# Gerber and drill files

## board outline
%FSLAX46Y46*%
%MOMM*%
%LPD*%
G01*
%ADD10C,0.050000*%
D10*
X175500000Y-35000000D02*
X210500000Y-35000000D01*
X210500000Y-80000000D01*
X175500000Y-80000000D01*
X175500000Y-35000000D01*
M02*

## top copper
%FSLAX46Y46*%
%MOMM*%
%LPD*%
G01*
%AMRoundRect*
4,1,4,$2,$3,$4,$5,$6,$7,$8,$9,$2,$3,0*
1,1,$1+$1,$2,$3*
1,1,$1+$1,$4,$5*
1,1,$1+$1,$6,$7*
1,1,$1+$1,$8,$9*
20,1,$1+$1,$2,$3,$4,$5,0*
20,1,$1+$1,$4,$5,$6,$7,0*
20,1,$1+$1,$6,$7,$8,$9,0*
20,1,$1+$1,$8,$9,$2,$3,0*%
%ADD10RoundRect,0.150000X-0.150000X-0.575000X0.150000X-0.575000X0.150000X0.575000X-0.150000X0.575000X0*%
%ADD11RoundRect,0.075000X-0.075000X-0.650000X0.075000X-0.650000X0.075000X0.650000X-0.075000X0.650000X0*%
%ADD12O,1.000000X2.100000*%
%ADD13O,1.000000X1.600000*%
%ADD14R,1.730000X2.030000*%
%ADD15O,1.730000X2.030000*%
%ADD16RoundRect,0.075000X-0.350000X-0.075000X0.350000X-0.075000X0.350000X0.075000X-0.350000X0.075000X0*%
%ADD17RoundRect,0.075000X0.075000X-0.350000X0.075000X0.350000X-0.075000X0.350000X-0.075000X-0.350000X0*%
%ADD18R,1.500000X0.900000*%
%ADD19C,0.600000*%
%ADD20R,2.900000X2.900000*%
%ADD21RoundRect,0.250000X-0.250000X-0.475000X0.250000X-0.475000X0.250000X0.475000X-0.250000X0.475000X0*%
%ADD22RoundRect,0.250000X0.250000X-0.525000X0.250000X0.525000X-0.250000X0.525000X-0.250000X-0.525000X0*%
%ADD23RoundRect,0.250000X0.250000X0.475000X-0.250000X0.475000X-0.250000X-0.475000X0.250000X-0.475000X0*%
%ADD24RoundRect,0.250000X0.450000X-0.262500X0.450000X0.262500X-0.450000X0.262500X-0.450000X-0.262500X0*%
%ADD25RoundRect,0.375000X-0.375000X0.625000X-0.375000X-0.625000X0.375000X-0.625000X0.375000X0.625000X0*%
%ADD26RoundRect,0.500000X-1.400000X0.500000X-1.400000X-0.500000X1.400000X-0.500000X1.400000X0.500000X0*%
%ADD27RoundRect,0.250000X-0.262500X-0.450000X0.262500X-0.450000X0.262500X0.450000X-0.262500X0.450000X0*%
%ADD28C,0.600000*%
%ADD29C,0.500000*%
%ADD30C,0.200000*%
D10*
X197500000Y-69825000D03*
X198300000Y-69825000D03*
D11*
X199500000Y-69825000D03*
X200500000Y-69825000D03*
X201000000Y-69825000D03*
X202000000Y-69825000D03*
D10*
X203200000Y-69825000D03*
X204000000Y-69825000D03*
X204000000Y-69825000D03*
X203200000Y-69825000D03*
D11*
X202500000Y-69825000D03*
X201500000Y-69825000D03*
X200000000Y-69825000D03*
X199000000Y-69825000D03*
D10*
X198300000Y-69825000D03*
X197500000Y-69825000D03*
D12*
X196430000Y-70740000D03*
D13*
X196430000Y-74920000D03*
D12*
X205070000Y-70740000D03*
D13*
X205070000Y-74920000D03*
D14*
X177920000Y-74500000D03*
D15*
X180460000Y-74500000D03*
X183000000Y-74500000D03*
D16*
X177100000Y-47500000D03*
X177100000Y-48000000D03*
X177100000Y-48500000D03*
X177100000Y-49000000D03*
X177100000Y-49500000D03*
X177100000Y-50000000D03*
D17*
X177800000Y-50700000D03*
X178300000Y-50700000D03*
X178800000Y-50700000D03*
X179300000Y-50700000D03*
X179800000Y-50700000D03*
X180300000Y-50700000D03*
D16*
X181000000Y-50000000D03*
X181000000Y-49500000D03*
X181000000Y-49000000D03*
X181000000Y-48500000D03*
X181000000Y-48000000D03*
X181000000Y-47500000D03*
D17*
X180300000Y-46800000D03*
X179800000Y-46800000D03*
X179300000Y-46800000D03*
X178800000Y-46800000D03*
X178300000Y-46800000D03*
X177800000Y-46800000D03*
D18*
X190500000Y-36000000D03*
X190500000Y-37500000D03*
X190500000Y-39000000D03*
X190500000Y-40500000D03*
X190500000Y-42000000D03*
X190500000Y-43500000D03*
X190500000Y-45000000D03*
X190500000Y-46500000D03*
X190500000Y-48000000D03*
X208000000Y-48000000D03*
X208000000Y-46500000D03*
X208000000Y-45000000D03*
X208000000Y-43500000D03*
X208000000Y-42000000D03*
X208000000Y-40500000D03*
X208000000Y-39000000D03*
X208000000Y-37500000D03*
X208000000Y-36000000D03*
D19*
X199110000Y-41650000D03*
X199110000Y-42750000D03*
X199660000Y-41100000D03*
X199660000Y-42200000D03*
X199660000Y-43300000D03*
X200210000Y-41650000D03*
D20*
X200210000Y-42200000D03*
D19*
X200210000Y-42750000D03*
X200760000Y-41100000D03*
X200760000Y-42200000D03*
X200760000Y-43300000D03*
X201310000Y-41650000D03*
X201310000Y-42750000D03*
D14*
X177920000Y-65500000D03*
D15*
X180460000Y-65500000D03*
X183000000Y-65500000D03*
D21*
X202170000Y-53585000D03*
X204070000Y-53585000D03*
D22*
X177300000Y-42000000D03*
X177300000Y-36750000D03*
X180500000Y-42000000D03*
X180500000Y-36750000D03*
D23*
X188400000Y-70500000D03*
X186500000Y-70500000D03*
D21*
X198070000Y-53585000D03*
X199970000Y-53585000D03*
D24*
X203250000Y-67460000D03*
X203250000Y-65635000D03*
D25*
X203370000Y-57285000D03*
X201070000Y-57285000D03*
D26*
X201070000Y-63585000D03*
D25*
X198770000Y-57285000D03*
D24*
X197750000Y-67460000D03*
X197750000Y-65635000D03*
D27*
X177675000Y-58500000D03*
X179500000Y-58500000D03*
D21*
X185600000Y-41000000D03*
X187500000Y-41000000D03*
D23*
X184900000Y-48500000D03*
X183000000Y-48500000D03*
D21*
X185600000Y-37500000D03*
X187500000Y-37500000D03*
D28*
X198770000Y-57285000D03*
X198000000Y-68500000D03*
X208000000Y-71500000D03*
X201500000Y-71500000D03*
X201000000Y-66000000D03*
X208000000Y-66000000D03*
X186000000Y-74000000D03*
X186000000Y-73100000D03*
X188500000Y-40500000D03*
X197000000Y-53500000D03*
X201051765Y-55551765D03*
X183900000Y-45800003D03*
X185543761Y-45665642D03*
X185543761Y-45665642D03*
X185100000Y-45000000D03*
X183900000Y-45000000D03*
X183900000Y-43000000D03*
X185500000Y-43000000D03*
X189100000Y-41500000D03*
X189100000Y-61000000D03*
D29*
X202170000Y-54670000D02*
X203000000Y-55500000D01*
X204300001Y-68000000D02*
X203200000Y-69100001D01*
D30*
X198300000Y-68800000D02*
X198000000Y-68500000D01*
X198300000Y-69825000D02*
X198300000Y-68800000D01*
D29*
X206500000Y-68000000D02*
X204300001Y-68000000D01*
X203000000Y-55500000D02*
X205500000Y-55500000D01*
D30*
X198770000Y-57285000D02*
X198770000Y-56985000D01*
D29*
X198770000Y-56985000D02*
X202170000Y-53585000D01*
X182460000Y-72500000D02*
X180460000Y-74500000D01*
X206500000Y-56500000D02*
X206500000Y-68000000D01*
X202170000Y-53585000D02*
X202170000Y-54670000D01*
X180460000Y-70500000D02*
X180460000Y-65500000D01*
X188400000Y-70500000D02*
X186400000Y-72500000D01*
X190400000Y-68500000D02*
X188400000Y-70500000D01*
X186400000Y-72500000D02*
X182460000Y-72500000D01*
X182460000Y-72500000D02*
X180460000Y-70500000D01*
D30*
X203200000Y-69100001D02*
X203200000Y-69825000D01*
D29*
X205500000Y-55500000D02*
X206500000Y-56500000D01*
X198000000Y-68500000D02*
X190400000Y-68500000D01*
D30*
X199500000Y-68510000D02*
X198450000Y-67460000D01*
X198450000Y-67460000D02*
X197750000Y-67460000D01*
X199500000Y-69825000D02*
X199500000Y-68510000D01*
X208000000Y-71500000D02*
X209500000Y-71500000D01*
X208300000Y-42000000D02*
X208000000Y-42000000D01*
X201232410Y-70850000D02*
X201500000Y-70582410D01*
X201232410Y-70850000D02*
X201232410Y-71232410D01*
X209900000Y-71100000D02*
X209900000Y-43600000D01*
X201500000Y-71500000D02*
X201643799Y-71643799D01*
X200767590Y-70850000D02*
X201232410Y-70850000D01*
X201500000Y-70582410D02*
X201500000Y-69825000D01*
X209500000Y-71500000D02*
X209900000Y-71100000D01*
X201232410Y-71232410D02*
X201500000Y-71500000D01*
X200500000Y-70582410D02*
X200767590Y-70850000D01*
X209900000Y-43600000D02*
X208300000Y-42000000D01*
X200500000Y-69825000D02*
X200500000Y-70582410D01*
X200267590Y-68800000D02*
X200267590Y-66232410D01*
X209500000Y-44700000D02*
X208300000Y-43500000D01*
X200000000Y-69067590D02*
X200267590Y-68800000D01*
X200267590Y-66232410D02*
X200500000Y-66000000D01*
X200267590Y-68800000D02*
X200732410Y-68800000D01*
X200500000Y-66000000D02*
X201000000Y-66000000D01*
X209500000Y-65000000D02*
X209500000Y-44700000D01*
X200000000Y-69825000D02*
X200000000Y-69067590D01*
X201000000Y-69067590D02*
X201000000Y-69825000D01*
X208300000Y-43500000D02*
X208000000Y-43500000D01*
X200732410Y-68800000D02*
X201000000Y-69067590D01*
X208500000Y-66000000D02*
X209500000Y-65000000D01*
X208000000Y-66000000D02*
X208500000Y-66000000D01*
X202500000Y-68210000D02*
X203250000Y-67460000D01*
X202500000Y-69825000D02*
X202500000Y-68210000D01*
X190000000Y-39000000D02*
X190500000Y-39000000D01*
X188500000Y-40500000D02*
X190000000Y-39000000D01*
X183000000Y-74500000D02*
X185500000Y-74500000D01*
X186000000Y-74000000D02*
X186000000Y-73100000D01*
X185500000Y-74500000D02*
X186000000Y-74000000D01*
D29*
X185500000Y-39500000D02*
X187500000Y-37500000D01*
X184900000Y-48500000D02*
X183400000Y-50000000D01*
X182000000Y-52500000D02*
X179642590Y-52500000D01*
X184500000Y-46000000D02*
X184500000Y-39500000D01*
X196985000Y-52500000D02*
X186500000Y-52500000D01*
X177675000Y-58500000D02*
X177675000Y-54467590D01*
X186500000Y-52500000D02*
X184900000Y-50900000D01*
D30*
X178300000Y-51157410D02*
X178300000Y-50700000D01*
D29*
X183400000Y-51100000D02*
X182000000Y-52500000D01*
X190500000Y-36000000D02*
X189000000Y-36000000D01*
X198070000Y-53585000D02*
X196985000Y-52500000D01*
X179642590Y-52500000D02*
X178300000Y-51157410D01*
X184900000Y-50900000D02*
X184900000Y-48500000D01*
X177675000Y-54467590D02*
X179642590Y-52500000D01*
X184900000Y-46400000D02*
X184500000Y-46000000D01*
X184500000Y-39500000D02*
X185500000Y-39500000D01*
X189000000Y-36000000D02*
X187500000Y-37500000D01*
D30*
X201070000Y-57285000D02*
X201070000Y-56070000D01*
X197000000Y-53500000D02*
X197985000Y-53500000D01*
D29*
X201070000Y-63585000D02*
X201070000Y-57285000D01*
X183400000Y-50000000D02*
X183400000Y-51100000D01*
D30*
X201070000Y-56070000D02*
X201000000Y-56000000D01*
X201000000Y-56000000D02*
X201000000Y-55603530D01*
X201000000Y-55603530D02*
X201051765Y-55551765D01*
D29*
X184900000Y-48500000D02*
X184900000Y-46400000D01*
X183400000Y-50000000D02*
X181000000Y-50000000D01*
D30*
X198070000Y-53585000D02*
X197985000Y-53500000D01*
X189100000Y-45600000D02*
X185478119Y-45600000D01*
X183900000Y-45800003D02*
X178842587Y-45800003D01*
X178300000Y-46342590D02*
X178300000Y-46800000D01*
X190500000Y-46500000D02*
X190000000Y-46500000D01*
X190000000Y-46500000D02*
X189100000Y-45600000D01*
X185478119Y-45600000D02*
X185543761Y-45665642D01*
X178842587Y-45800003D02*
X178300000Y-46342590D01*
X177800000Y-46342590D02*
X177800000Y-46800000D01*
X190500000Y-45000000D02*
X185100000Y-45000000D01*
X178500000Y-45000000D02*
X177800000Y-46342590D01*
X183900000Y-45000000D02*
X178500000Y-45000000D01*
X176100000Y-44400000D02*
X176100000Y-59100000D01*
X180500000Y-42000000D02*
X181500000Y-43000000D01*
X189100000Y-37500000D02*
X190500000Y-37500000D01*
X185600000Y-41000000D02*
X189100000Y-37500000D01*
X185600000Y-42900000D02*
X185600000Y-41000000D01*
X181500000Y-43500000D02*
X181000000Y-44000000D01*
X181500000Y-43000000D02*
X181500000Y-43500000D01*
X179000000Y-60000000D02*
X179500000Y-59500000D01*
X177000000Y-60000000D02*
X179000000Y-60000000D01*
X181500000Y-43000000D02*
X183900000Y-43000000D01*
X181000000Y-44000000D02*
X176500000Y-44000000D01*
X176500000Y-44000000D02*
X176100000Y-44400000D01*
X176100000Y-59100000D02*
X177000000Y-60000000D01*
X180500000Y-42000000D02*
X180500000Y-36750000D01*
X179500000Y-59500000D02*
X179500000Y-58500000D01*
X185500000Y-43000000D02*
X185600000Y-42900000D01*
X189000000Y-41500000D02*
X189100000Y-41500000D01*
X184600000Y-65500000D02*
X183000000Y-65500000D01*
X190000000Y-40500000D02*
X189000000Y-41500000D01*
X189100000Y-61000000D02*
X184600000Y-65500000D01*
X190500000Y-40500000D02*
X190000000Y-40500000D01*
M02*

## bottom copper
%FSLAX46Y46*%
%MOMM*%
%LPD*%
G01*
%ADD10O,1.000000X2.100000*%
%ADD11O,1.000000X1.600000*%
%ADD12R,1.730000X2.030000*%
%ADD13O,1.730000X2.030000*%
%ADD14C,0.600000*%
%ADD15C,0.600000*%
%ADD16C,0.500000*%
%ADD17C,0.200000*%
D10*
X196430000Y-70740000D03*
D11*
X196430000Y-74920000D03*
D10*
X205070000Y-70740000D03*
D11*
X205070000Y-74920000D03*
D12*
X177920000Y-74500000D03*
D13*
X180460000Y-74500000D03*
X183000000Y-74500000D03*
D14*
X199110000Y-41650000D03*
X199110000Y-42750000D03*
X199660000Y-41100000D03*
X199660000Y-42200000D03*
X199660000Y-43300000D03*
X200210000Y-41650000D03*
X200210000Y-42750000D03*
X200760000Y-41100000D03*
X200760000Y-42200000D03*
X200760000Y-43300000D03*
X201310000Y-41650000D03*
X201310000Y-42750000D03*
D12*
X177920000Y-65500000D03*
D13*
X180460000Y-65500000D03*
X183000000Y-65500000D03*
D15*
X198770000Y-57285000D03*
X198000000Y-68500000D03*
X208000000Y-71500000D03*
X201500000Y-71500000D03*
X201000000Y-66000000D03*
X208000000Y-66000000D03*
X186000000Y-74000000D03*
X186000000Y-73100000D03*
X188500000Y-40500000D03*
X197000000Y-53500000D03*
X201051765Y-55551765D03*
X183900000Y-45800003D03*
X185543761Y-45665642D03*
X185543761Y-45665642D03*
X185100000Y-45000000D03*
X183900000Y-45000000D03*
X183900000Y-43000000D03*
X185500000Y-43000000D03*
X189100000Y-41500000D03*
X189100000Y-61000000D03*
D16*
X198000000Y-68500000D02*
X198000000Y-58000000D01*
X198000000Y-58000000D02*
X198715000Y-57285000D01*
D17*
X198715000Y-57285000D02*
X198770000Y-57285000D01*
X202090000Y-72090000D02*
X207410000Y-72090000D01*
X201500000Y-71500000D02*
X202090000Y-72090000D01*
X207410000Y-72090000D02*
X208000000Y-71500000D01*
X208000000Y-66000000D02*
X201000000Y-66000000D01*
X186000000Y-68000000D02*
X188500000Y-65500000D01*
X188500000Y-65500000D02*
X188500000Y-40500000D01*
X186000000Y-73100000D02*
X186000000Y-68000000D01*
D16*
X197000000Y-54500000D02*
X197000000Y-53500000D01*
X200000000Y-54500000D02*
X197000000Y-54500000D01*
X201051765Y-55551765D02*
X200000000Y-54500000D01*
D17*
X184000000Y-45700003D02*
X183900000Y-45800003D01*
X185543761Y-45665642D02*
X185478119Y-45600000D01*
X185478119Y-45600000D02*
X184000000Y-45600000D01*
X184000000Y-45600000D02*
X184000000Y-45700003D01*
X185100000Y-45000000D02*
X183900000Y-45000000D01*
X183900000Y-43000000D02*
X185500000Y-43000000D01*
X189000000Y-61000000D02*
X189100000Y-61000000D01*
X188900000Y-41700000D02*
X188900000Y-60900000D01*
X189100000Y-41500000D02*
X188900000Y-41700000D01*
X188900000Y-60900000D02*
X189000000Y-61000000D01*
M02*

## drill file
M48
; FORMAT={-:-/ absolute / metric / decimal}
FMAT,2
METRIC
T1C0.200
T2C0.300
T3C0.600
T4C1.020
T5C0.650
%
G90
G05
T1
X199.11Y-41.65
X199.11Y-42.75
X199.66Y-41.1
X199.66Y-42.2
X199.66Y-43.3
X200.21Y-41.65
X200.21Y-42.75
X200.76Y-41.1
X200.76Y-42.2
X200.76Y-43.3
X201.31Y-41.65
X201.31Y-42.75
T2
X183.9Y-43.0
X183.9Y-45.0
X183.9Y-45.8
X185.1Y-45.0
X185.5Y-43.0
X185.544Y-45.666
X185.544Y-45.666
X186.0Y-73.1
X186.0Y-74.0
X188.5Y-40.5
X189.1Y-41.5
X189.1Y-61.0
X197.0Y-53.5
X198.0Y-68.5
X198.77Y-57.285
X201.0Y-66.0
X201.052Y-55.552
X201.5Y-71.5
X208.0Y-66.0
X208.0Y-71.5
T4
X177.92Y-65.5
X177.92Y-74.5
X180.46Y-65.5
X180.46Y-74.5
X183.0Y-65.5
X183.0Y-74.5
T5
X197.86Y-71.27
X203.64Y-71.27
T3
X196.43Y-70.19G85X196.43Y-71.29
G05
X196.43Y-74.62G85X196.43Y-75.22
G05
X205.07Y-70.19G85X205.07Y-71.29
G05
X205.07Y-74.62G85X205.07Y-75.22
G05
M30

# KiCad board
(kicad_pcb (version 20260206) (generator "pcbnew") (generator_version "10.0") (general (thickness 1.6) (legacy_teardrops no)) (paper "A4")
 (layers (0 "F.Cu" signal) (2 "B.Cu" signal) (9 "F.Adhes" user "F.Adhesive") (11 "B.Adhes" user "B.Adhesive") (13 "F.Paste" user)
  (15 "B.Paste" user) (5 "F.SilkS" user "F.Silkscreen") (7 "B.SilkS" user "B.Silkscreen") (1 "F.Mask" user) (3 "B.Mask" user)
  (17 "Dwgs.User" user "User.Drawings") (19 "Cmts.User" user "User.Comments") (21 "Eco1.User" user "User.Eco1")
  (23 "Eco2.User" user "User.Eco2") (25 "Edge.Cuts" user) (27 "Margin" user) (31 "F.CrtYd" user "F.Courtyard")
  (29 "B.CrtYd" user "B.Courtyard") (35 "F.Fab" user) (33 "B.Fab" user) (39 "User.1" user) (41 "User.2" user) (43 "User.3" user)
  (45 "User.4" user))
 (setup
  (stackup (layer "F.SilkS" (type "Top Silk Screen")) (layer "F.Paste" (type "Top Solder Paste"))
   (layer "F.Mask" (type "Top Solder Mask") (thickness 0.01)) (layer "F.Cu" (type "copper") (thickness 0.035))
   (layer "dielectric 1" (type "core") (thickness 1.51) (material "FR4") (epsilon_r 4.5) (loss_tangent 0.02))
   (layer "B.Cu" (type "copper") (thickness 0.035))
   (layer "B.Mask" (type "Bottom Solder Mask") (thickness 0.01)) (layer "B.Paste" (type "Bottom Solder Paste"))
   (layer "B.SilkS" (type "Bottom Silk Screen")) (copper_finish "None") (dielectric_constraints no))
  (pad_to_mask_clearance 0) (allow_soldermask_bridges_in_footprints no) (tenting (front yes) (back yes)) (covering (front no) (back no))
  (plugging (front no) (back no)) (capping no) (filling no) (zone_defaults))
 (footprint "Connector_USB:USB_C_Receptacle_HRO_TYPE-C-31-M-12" (layer "F.Cu") (at 200.75 73.87)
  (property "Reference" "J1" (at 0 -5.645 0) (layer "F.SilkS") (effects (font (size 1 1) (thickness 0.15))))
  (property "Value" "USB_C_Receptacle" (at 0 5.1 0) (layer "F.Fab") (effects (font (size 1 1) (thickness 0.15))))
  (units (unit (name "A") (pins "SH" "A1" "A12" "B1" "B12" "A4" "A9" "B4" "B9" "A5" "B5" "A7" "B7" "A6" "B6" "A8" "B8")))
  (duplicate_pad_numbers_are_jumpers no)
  (pad "" np_thru_hole circle (at -2.89 -2.6) (size 0.65 0.65) (drill 0.65) (layers "*.Cu" "*.Mask"))
  (pad "" np_thru_hole circle (at 2.89 -2.6) (size 0.65 0.65) (drill 0.65) (layers "*.Cu" "*.Mask"))
  (pad "A1" smd roundrect (at -3.25 -4.045) (size 0.6 1.45) (layers "F.Cu" "F.Mask" "F.Paste") (roundrect_rratio 0.25)
   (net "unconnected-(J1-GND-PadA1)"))
  (pad "A4" smd roundrect (at -2.45 -4.045) (size 0.6 1.45) (layers "F.Cu" "F.Mask" "F.Paste") (roundrect_rratio 0.25) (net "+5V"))
  (pad "A5" smd roundrect (at -1.25 -4.045) (size 0.3 1.45) (layers "F.Cu" "F.Mask" "F.Paste") (roundrect_rratio 0.25) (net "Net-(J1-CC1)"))
  (pad "A6" smd roundrect (at -0.25 -4.045) (size 0.3 1.45) (layers "F.Cu" "F.Mask" "F.Paste") (roundrect_rratio 0.25) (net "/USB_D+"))
  (pad "A7" smd roundrect (at 0.25 -4.045) (size 0.3 1.45) (layers "F.Cu" "F.Mask" "F.Paste") (roundrect_rratio 0.25) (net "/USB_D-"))
  (pad "A8" smd roundrect (at 1.25 -4.045) (size 0.3 1.45) (layers "F.Cu" "F.Mask" "F.Paste") (roundrect_rratio 0.25)
   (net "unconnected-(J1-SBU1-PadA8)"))
  (pad "A9" smd roundrect (at 2.45 -4.045) (size 0.6 1.45) (layers "F.Cu" "F.Mask" "F.Paste") (roundrect_rratio 0.25) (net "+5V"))
  (pad "A12" smd roundrect (at 3.25 -4.045) (size 0.6 1.45) (layers "F.Cu" "F.Mask" "F.Paste") (roundrect_rratio 0.25)
   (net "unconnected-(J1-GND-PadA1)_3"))
  (pad "B1" smd roundrect (at 3.25 -4.045) (size 0.6 1.45) (layers "F.Cu" "F.Mask" "F.Paste") (roundrect_rratio 0.25)
   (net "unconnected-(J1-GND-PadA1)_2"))
  (pad "B4" smd roundrect (at 2.45 -4.045) (size 0.6 1.45) (layers "F.Cu" "F.Mask" "F.Paste") (roundrect_rratio 0.25) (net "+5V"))
  (pad "B5" smd roundrect (at 1.75 -4.045) (size 0.3 1.45) (layers "F.Cu" "F.Mask" "F.Paste") (roundrect_rratio 0.25) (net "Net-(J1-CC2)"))
  (pad "B6" smd roundrect (at 0.75 -4.045) (size 0.3 1.45) (layers "F.Cu" "F.Mask" "F.Paste") (roundrect_rratio 0.25) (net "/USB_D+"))
  (pad "B7" smd roundrect (at -0.75 -4.045) (size 0.3 1.45) (layers "F.Cu" "F.Mask" "F.Paste") (roundrect_rratio 0.25) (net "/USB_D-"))
  (pad "B8" smd roundrect (at -1.75 -4.045) (size 0.3 1.45) (layers "F.Cu" "F.Mask" "F.Paste") (roundrect_rratio 0.25)
   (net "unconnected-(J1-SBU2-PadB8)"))
  (pad "B9" smd roundrect (at -2.45 -4.045) (size 0.6 1.45) (layers "F.Cu" "F.Mask" "F.Paste") (roundrect_rratio 0.25) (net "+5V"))
  (pad "B12" smd roundrect (at -3.25 -4.045) (size 0.6 1.45) (layers "F.Cu" "F.Mask" "F.Paste") (roundrect_rratio 0.25)
   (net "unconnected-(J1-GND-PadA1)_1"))
  (pad "SH" thru_hole oval (at -4.32 -3.13) (size 1 2.1) (drill oval 0.6 1.7) (layers "*.Cu" "*.Mask") (remove_unused_layers no)
   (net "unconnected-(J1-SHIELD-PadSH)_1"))
  (pad "SH" thru_hole oval (at -4.32 1.05) (size 1 1.6) (drill oval 0.6 1.2) (layers "*.Cu" "*.Mask") (remove_unused_layers no)
   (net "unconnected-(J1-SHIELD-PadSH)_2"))
  (pad "SH" thru_hole oval (at 4.32 -3.13) (size 1 2.1) (drill oval 0.6 1.7) (layers "*.Cu" "*.Mask") (remove_unused_layers no)
   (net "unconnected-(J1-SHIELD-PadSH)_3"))
  (pad "SH" thru_hole oval (at 4.32 1.05) (size 1 1.6) (drill oval 0.6 1.2) (layers "*.Cu" "*.Mask") (remove_unused_layers no)
   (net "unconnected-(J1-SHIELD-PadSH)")))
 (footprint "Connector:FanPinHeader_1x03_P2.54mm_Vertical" (layer "F.Cu") (at 177.92 74.5)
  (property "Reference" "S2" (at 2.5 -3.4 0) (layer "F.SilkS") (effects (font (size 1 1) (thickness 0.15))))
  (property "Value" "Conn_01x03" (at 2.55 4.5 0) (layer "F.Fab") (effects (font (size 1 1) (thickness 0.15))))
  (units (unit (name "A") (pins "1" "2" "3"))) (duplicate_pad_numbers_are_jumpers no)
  (pad "1" thru_hole rect (at 0 0 90) (size 2.03 1.73) (drill 1.02) (layers "*.Cu" "*.Mask") (remove_unused_layers no) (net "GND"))
  (pad "2" thru_hole oval (at 2.54 0 90) (size 2.03 1.73) (drill 1.02) (layers "*.Cu" "*.Mask") (remove_unused_layers no) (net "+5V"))
  (pad "3" thru_hole oval (at 5.08 0 90) (size 2.03 1.73) (drill 1.02) (layers "*.Cu" "*.Mask") (remove_unused_layers no) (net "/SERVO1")))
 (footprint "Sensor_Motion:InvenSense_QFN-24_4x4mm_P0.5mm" (layer "F.Cu") (at 179.05 48.75)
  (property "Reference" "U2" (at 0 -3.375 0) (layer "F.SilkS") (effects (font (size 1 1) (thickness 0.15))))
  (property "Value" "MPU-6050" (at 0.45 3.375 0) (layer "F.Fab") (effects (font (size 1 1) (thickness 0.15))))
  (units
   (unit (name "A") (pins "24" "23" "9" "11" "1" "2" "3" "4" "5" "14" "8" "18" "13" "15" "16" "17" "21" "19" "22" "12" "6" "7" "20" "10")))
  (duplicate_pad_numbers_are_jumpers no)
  (pad "1" smd roundrect (at -1.95 -1.25) (size 0.85 0.3) (layers "F.Cu" "F.Mask" "F.Paste") (roundrect_rratio 0.25)
   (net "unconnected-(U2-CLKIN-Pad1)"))
  (pad "2" smd roundrect (at -1.95 -0.75) (size 0.85 0.3) (layers "F.Cu" "F.Mask" "F.Paste") (roundrect_rratio 0.25)
   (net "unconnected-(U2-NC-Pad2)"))
  (pad "3" smd roundrect (at -1.95 -0.25) (size 0.85 0.3) (layers "F.Cu" "F.Mask" "F.Paste") (roundrect_rratio 0.25)
   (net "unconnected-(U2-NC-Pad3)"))
  (pad "4" smd roundrect (at -1.95 0.25) (size 0.85 0.3) (layers "F.Cu" "F.Mask" "F.Paste") (roundrect_rratio 0.25)
   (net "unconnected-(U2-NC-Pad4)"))
  (pad "5" smd roundrect (at -1.95 0.75) (size 0.85 0.3) (layers "F.Cu" "F.Mask" "F.Paste") (roundrect_rratio 0.25)
   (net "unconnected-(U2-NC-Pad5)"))
  (pad "6" smd roundrect (at -1.95 1.25) (size 0.85 0.3) (layers "F.Cu" "F.Mask" "F.Paste") (roundrect_rratio 0.25)
   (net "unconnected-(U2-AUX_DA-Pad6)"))
  (pad "7" smd roundrect (at -1.25 1.95 90) (size 0.85 0.3) (layers "F.Cu" "F.Mask" "F.Paste") (roundrect_rratio 0.25)
   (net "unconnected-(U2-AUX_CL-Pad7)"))
  (pad "8" smd roundrect (at -0.75 1.95 90) (size 0.85 0.3) (layers "F.Cu" "F.Mask" "F.Paste") (roundrect_rratio 0.25) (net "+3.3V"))
  (pad "9" smd roundrect (at -0.25 1.95 90) (size 0.85 0.3) (layers "F.Cu" "F.Mask" "F.Paste") (roundrect_rratio 0.25)
   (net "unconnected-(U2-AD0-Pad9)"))
  (pad "10" smd roundrect (at 0.25 1.95 90) (size 0.85 0.3) (layers "F.Cu" "F.Mask" "F.Paste") (roundrect_rratio 0.25)
   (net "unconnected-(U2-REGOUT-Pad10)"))
  (pad "11" smd roundrect (at 0.75 1.95 90) (size 0.85 0.3) (layers "F.Cu" "F.Mask" "F.Paste") (roundrect_rratio 0.25)
   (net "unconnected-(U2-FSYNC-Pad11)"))
  (pad "12" smd roundrect (at 1.25 1.95 90) (size 0.85 0.3) (layers "F.Cu" "F.Mask" "F.Paste") (roundrect_rratio 0.25)
   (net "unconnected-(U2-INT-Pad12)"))
  (pad "13" smd roundrect (at 1.95 1.25) (size 0.85 0.3) (layers "F.Cu" "F.Mask" "F.Paste") (roundrect_rratio 0.25) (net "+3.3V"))
  (pad "14" smd roundrect (at 1.95 0.75) (size 0.85 0.3) (layers "F.Cu" "F.Mask" "F.Paste") (roundrect_rratio 0.25)
   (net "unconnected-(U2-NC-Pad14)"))
  (pad "15" smd roundrect (at 1.95 0.25) (size 0.85 0.3) (layers "F.Cu" "F.Mask" "F.Paste") (roundrect_rratio 0.25)
   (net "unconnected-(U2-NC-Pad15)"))
  (pad "16" smd roundrect (at 1.95 -0.25) (size 0.85 0.3) (layers "F.Cu" "F.Mask" "F.Paste") (roundrect_rratio 0.25)
   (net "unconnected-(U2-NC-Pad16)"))
  (pad "17" smd roundrect (at 1.95 -0.75) (size 0.85 0.3) (layers "F.Cu" "F.Mask" "F.Paste") (roundrect_rratio 0.25)
   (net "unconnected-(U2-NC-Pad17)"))
  (pad "18" smd roundrect (at 1.95 -1.25) (size 0.85 0.3) (layers "F.Cu" "F.Mask" "F.Paste") (roundrect_rratio 0.25) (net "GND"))
  (pad "19" smd roundrect (at 1.25 -1.95 90) (size 0.85 0.3) (layers "F.Cu" "F.Mask" "F.Paste") (roundrect_rratio 0.25)
   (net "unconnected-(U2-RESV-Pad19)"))
  (pad "20" smd roundrect (at 0.75 -1.95 90) (size 0.85 0.3) (layers "F.Cu" "F.Mask" "F.Paste") (roundrect_rratio 0.25)
   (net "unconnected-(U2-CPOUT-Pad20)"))
  (pad "21" smd roundrect (at 0.25 -1.95 90) (size 0.85 0.3) (layers "F.Cu" "F.Mask" "F.Paste") (roundrect_rratio 0.25)
   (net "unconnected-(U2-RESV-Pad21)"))
  (pad "22" smd roundrect (at -0.25 -1.95 90) (size 0.85 0.3) (layers "F.Cu" "F.Mask" "F.Paste") (roundrect_rratio 0.25)
   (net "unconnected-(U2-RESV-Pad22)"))
  (pad "23" smd roundrect (at -0.75 -1.95 90) (size 0.85 0.3) (layers "F.Cu" "F.Mask" "F.Paste") (roundrect_rratio 0.25) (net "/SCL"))
  (pad "24" smd roundrect (at -1.25 -1.95 90) (size 0.85 0.3) (layers "F.Cu" "F.Mask" "F.Paste") (roundrect_rratio 0.25) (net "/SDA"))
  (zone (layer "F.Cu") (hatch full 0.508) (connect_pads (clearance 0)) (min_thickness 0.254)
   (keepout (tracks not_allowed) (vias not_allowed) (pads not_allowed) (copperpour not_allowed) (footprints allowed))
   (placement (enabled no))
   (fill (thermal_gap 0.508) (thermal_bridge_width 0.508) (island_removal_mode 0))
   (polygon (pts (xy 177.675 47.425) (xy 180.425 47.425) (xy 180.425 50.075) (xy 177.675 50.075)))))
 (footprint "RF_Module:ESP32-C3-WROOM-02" (layer "F.Cu") (at 199.25 42)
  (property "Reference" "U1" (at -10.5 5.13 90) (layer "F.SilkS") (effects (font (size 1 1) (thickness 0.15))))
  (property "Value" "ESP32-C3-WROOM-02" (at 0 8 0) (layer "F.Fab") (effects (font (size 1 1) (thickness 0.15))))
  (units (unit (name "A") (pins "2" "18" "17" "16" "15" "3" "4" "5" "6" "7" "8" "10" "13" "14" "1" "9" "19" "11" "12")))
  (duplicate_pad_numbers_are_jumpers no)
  (pad "" smd rect (at -0.14 -0.9) (size 0.7 0.7) (layers "F.Paste"))
  (pad "" smd rect (at -0.14 0.2) (size 0.7 0.7) (layers "F.Paste"))
  (pad "" smd rect (at -0.14 1.3) (size 0.7 0.7) (layers "F.Paste"))
  (pad "" smd rect (at 0.96 -0.9) (size 0.7 0.7) (layers "F.Paste"))
  (pad "" smd rect (at 0.96 0.2) (size 0.7 0.7) (layers "F.Paste"))
  (pad "" smd rect (at 0.96 1.3) (size 0.7 0.7) (layers "F.Paste"))
  (pad "" smd rect (at 2.06 -0.9) (size 0.7 0.7) (layers "F.Paste"))
  (pad "" smd rect (at 2.06 0.2) (size 0.7 0.7) (layers "F.Paste"))
  (pad "" smd rect (at 2.06 1.3) (size 0.7 0.7) (layers "F.Paste"))
  (pad "1" smd rect (at -8.75 -6) (size 1.5 0.9) (layers "F.Cu" "F.Mask" "F.Paste") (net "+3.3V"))
  (pad "2" smd rect (at -8.75 -4.5) (size 1.5 0.9) (layers "F.Cu" "F.Mask" "F.Paste") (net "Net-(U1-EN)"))
  (pad "3" smd rect (at -8.75 -3) (size 1.5 0.9) (layers "F.Cu" "F.Mask" "F.Paste") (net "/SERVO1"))
  (pad "4" smd rect (at -8.75 -1.5) (size 1.5 0.9) (layers "F.Cu" "F.Mask" "F.Paste") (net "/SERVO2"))
  (pad "5" smd rect (at -8.75 0) (size 1.5 0.9) (layers "F.Cu" "F.Mask" "F.Paste") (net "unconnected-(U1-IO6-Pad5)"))
  (pad "6" smd rect (at -8.75 1.5) (size 1.5 0.9) (layers "F.Cu" "F.Mask" "F.Paste") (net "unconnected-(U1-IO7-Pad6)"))
  (pad "7" smd rect (at -8.75 3) (size 1.5 0.9) (layers "F.Cu" "F.Mask" "F.Paste") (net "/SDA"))
  (pad "8" smd rect (at -8.75 4.5) (size 1.5 0.9) (layers "F.Cu" "F.Mask" "F.Paste") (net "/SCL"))
  (pad "9" smd rect (at -8.75 6) (size 1.5 0.9) (layers "F.Cu" "F.Mask" "F.Paste") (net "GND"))
  (pad "10" smd rect (at 8.75 6) (size 1.5 0.9) (layers "F.Cu" "F.Mask" "F.Paste") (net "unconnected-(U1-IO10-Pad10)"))
  (pad "11" smd rect (at 8.75 4.5) (size 1.5 0.9) (layers "F.Cu" "F.Mask" "F.Paste") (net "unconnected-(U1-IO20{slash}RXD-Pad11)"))
  (pad "12" smd rect (at 8.75 3) (size 1.5 0.9) (layers "F.Cu" "F.Mask" "F.Paste") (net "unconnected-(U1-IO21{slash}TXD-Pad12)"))
  (pad "13" smd rect (at 8.75 1.5) (size 1.5 0.9) (layers "F.Cu" "F.Mask" "F.Paste") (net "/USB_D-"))
  (pad "14" smd rect (at 8.75 0) (size 1.5 0.9) (layers "F.Cu" "F.Mask" "F.Paste") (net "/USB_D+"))
  (pad "15" smd rect (at 8.75 -1.5) (size 1.5 0.9) (layers "F.Cu" "F.Mask" "F.Paste") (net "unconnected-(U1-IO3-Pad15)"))
  (pad "16" smd rect (at 8.75 -3) (size 1.5 0.9) (layers "F.Cu" "F.Mask" "F.Paste") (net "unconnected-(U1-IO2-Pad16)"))
  (pad "17" smd rect (at 8.75 -4.5) (size 1.5 0.9) (layers "F.Cu" "F.Mask" "F.Paste") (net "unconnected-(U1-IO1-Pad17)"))
  (pad "18" smd rect (at 8.75 -6) (size 1.5 0.9) (layers "F.Cu" "F.Mask" "F.Paste") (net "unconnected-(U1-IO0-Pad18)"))
  (pad "19" thru_hole circle (at -0.14 -0.35) (size 0.6 0.6) (drill 0.2) (layers "*.Cu" "F.Mask") (remove_unused_layers no) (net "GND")
   (zone_connect 2))
  (pad "19" thru_hole circle (at -0.14 0.75) (size 0.6 0.6) (drill 0.2) (layers "*.Cu" "F.Mask") (remove_unused_layers no) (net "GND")
   (zone_connect 2))
  (pad "19" thru_hole circle (at 0.41 -0.9) (size 0.6 0.6) (drill 0.2) (layers "*.Cu" "F.Mask") (remove_unused_layers no) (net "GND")
   (zone_connect 2))
  (pad "19" thru_hole circle (at 0.41 0.2) (size 0.6 0.6) (drill 0.2) (layers "*.Cu" "F.Mask") (remove_unused_layers no) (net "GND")
   (zone_connect 2))
  (pad "19" thru_hole circle (at 0.41 1.3) (size 0.6 0.6) (drill 0.2) (layers "*.Cu" "F.Mask") (remove_unused_layers no) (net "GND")
   (zone_connect 2))
  (pad "19" thru_hole circle (at 0.96 -0.35) (size 0.6 0.6) (drill 0.2) (layers "*.Cu" "F.Mask") (remove_unused_layers no) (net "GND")
   (zone_connect 2))
  (pad "19" smd rect (at 0.96 0.2) (size 2.9 2.9) (layers "F.Cu" "F.Mask") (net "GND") (zone_connect 2))
  (pad "19" thru_hole circle (at 0.96 0.75) (size 0.6 0.6) (drill 0.2) (layers "*.Cu" "F.Mask") (remove_unused_layers no) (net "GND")
   (zone_connect 2))
  (pad "19" thru_hole circle (at 1.51 -0.9) (size 0.6 0.6) (drill 0.2) (layers "*.Cu" "F.Mask") (remove_unused_layers no) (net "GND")
   (zone_connect 2))
  (pad "19" thru_hole circle (at 1.51 0.2) (size 0.6 0.6) (drill 0.2) (layers "*.Cu" "F.Mask") (remove_unused_layers no) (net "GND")
   (zone_connect 2))
  (pad "19" thru_hole circle (at 1.51 1.3) (size 0.6 0.6) (drill 0.2) (layers "*.Cu" "F.Mask") (remove_unused_layers no) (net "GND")
   (zone_connect 2))
  (pad "19" thru_hole circle (at 2.06 -0.35) (size 0.6 0.6) (drill 0.2) (layers "*.Cu" "F.Mask") (remove_unused_layers no) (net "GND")
   (zone_connect 2))
  (pad "19" thru_hole circle (at 2.06 0.75) (size 0.6 0.6) (drill 0.2) (layers "*.Cu" "F.Mask") (remove_unused_layers no) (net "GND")
   (zone_connect 2))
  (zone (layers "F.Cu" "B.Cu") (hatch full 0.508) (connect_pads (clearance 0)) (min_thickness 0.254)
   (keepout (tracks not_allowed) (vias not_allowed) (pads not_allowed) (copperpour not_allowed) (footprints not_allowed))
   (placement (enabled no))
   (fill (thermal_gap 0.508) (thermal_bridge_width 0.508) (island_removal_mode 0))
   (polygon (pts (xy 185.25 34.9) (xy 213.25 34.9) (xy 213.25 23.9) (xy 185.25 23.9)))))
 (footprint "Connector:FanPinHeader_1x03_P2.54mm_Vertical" (layer "F.Cu") (at 177.92 65.5)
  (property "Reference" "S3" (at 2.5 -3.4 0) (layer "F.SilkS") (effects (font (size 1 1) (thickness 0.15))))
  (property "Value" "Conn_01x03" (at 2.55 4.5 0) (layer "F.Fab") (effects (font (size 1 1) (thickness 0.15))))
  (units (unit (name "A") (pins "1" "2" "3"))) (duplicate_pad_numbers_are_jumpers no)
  (pad "1" thru_hole rect (at 0 0 90) (size 2.03 1.73) (drill 1.02) (layers "*.Cu" "*.Mask") (remove_unused_layers no) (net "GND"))
  (pad "2" thru_hole oval (at 2.54 0 90) (size 2.03 1.73) (drill 1.02) (layers "*.Cu" "*.Mask") (remove_unused_layers no) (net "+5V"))
  (pad "3" thru_hole oval (at 5.08 0 90) (size 2.03 1.73) (drill 1.02) (layers "*.Cu" "*.Mask") (remove_unused_layers no) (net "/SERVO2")))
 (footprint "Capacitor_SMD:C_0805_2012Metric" (layer "F.Cu") (at 203.12 53.585)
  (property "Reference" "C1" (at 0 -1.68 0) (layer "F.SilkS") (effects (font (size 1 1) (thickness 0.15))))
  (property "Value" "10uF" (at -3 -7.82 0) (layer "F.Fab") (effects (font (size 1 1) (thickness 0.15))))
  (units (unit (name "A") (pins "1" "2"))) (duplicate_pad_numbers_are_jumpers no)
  (pad "1" smd roundrect (at -0.95 0) (size 1 1.45) (layers "F.Cu" "F.Mask" "F.Paste") (roundrect_rratio 0.25) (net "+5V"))
  (pad "2" smd roundrect (at 0.95 0) (size 1 1.45) (layers "F.Cu" "F.Mask" "F.Paste") (roundrect_rratio 0.25) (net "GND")))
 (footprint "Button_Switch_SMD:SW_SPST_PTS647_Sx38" (layer "F.Cu") (at 178.9 39.375 90)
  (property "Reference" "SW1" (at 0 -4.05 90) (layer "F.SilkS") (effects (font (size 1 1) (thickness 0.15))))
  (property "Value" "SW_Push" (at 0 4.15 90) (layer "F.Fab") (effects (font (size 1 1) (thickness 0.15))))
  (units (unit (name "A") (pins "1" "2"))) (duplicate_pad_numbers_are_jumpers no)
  (pad "1" smd roundrect (at -2.625 -1.6 90) (size 1.55 1) (layers "F.Cu" "F.Mask" "F.Paste") (roundrect_rratio 0.25) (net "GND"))
  (pad "1" smd roundrect (at 2.625 -1.6 90) (size 1.55 1) (layers "F.Cu" "F.Mask" "F.Paste") (roundrect_rratio 0.25) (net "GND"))
  (pad "2" smd roundrect (at -2.625 1.6 90) (size 1.55 1) (layers "F.Cu" "F.Mask" "F.Paste") (roundrect_rratio 0.25) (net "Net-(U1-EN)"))
  (pad "2" smd roundrect (at 2.625 1.6 90) (size 1.55 1) (layers "F.Cu" "F.Mask" "F.Paste") (roundrect_rratio 0.25) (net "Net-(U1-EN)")))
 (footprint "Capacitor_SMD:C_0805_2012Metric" (layer "F.Cu") (at 187.45 70.5 180)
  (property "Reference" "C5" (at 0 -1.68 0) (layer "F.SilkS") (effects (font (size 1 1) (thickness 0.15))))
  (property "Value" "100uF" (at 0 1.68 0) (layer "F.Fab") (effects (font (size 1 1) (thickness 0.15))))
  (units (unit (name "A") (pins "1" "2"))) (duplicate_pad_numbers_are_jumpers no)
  (pad "1" smd roundrect (at -0.95 0 180) (size 1 1.45) (layers "F.Cu" "F.Mask" "F.Paste") (roundrect_rratio 0.25) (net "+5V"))
  (pad "2" smd roundrect (at 0.95 0 180) (size 1 1.45) (layers "F.Cu" "F.Mask" "F.Paste") (roundrect_rratio 0.25) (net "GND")))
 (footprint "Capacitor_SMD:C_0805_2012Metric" (layer "F.Cu") (at 199.02 53.585)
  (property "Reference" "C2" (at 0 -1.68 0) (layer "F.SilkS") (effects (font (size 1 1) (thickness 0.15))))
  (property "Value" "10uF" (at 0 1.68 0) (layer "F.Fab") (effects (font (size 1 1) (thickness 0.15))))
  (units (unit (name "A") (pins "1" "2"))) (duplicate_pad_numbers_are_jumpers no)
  (pad "1" smd roundrect (at -0.95 0) (size 1 1.45) (layers "F.Cu" "F.Mask" "F.Paste") (roundrect_rratio 0.25) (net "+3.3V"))
  (pad "2" smd roundrect (at 0.95 0) (size 1 1.45) (layers "F.Cu" "F.Mask" "F.Paste") (roundrect_rratio 0.25) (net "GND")))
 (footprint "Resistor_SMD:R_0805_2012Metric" (layer "F.Cu") (at 203.25 66.5475 90)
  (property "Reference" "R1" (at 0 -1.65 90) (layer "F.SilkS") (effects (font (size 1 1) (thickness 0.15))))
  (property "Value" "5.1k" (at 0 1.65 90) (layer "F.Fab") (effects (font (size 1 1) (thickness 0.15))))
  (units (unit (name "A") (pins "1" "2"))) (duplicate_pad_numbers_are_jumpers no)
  (pad "1" smd roundrect (at -0.9125 0 90) (size 1.025 1.4) (layers "F.Cu" "F.Mask" "F.Paste") (roundrect_rratio 0.243902)
   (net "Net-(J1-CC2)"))
  (pad "2" smd roundrect (at 0.9125 0 90) (size 1.025 1.4) (layers "F.Cu" "F.Mask" "F.Paste") (roundrect_rratio 0.243902) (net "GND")))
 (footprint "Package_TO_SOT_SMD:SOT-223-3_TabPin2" (layer "F.Cu") (at 201.07 60.435 -90)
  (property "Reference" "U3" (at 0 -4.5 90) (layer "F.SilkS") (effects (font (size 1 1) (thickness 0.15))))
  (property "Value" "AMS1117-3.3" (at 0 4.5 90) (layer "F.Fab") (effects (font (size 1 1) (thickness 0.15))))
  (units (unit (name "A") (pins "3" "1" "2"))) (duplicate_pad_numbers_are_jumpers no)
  (pad "1" smd roundrect (at -3.15 -2.3 270) (size 2 1.5) (layers "F.Cu" "F.Mask" "F.Paste") (roundrect_rratio 0.25) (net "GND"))
  (pad "2" smd roundrect (at -3.15 0 270) (size 2 1.5) (layers "F.Cu" "F.Mask" "F.Paste") (roundrect_rratio 0.25) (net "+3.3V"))
  (pad "2" smd roundrect (at 3.15 0 270) (size 2 3.8) (layers "F.Cu" "F.Mask" "F.Paste") (roundrect_rratio 0.25) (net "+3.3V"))
  (pad "3" smd roundrect (at -3.15 2.3 270) (size 2 1.5) (layers "F.Cu" "F.Mask" "F.Paste") (roundrect_rratio 0.25) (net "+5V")))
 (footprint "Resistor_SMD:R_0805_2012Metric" (layer "F.Cu") (at 197.75 66.5475 90)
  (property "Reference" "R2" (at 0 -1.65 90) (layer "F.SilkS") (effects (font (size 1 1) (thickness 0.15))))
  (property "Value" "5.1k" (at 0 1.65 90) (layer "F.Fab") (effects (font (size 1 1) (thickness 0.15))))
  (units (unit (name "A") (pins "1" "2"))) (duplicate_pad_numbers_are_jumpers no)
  (pad "1" smd roundrect (at -0.9125 0 90) (size 1.025 1.4) (layers "F.Cu" "F.Mask" "F.Paste") (roundrect_rratio 0.243902)
   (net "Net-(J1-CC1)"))
  (pad "2" smd roundrect (at 0.9125 0 90) (size 1.025 1.4) (layers "F.Cu" "F.Mask" "F.Paste") (roundrect_rratio 0.243902) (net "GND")))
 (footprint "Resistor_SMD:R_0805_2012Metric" (layer "F.Cu") (at 178.5875 58.5)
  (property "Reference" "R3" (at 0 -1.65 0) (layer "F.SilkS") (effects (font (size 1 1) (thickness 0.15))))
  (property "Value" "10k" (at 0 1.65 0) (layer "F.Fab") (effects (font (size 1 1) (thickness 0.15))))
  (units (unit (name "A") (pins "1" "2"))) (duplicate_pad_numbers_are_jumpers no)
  (pad "1" smd roundrect (at -0.9125 0) (size 1.025 1.4) (layers "F.Cu" "F.Mask" "F.Paste") (roundrect_rratio 0.243902) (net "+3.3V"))
  (pad "2" smd roundrect (at 0.9125 0) (size 1.025 1.4) (layers "F.Cu" "F.Mask" "F.Paste") (roundrect_rratio 0.243902) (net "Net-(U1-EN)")))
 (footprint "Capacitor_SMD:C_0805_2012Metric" (layer "F.Cu") (at 186.55 41)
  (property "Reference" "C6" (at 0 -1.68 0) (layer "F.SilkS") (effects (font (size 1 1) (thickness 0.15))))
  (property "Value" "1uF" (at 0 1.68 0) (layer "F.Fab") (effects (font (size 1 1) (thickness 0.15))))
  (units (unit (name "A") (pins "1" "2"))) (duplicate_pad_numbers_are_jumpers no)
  (pad "1" smd roundrect (at -0.95 0) (size 1 1.45) (layers "F.Cu" "F.Mask" "F.Paste") (roundrect_rratio 0.25) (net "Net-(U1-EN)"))
  (pad "2" smd roundrect (at 0.95 0) (size 1 1.45) (layers "F.Cu" "F.Mask" "F.Paste") (roundrect_rratio 0.25) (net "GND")))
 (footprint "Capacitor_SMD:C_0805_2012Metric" (layer "F.Cu") (at 183.95 48.5 180)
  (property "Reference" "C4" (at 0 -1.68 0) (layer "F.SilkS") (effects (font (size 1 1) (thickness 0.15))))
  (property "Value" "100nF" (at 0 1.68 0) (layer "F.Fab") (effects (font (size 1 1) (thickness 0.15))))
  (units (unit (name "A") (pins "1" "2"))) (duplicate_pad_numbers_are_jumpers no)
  (pad "1" smd roundrect (at -0.95 0 180) (size 1 1.45) (layers "F.Cu" "F.Mask" "F.Paste") (roundrect_rratio 0.25) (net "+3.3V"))
  (pad "2" smd roundrect (at 0.95 0 180) (size 1 1.45) (layers "F.Cu" "F.Mask" "F.Paste") (roundrect_rratio 0.25) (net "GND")))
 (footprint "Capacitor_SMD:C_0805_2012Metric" (layer "F.Cu") (at 186.55 37.5)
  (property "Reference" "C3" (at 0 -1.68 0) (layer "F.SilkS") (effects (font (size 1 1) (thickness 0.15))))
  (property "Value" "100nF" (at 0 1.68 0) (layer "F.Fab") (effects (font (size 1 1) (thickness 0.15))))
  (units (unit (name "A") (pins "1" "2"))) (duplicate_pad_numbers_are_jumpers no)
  (pad "1" smd roundrect (at -0.95 0) (size 1 1.45) (layers "F.Cu" "F.Mask" "F.Paste") (roundrect_rratio 0.25) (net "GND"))
  (pad "2" smd roundrect (at 0.95 0) (size 1 1.45) (layers "F.Cu" "F.Mask" "F.Paste") (roundrect_rratio 0.25) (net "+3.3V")))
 (gr_rect (start 175.5 35) (end 210.5 80) (stroke (width 0.05) (type default)) (fill no) (layer "Edge.Cuts"))
 (segment (start 202.17 54.67) (end 203 55.5) (width 0.5) (layer "F.Cu") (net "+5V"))
 (segment (start 204.300001 68) (end 203.2 69.100001) (width 0.5) (layer "F.Cu") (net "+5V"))
 (segment (start 198.3 68.8) (end 198 68.5) (width 0.2) (layer "F.Cu") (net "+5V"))
 (segment (start 198.3 69.825) (end 198.3 68.8) (width 0.2) (layer "F.Cu") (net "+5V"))
 (segment (start 206.5 68) (end 204.300001 68) (width 0.5) (layer "F.Cu") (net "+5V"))
 (segment (start 203 55.5) (end 205.5 55.5) (width 0.5) (layer "F.Cu") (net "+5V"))
 (segment (start 198.77 57.285) (end 198.77 56.985) (width 0.2) (layer "F.Cu") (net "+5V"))
 (segment (start 198.77 56.985) (end 202.17 53.585) (width 0.5) (layer "F.Cu") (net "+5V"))
 (segment (start 182.46 72.5) (end 180.46 74.5) (width 0.5) (layer "F.Cu") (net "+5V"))
 (segment (start 206.5 56.5) (end 206.5 68) (width 0.5) (layer "F.Cu") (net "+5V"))
 (segment (start 202.17 53.585) (end 202.17 54.67) (width 0.5) (layer "F.Cu") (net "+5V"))
 (segment (start 180.46 70.5) (end 180.46 65.5) (width 0.5) (layer "F.Cu") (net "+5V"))
 (segment (start 188.4 70.5) (end 186.4 72.5) (width 0.5) (layer "F.Cu") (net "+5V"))
 (segment (start 190.4 68.5) (end 188.4 70.5) (width 0.5) (layer "F.Cu") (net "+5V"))
 (segment (start 186.4 72.5) (end 182.46 72.5) (width 0.5) (layer "F.Cu") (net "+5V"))
 (segment (start 182.46 72.5) (end 180.46 70.5) (width 0.5) (layer "F.Cu") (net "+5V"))
 (segment (start 203.2 69.100001) (end 203.2 69.825) (width 0.2) (layer "F.Cu") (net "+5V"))
 (segment (start 205.5 55.5) (end 206.5 56.5) (width 0.5) (layer "F.Cu") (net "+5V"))
 (segment (start 198 68.5) (end 190.4 68.5) (width 0.5) (layer "F.Cu") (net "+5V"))
 (via (at 198.77 57.285) (size 0.6) (drill 0.3) (layers "F.Cu" "B.Cu") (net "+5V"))
 (via (at 198 68.5) (size 0.6) (drill 0.3) (layers "F.Cu" "B.Cu") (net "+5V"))
 (segment (start 198 68.5) (end 198 58) (width 0.5) (layer "B.Cu") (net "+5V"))
 (segment (start 198 58) (end 198.715 57.285) (width 0.5) (layer "B.Cu") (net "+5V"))
 (segment (start 198.715 57.285) (end 198.77 57.285) (width 0.2) (layer "B.Cu") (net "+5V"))
 (segment (start 199.5 68.51) (end 198.45 67.46) (width 0.2) (layer "F.Cu") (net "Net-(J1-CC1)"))
 (segment (start 198.45 67.46) (end 197.75 67.46) (width 0.2) (layer "F.Cu") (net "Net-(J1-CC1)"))
 (segment (start 199.5 69.825) (end 199.5 68.51) (width 0.2) (layer "F.Cu") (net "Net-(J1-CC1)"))
 (segment (start 208 71.5) (end 209.5 71.5) (width 0.2) (layer "F.Cu") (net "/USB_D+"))
 (segment (start 208.3 42) (end 208 42) (width 0.2) (layer "F.Cu") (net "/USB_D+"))
 (segment (start 201.23241 70.85) (end 201.5 70.58241) (width 0.2) (layer "F.Cu") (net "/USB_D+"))
 (segment (start 201.23241 70.85) (end 201.23241 71.23241) (width 0.2) (layer "F.Cu") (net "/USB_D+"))
 (segment (start 209.9 71.1) (end 209.9 43.6) (width 0.2) (layer "F.Cu") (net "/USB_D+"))
 (segment (start 201.5 71.5) (end 201.643799 71.643799) (width 0.2) (layer "F.Cu") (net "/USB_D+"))
 (segment (start 200.76759 70.85) (end 201.23241 70.85) (width 0.2) (layer "F.Cu") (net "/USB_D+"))
 (segment (start 201.5 70.58241) (end 201.5 69.825) (width 0.2) (layer "F.Cu") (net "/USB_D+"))
 (segment (start 209.5 71.5) (end 209.9 71.1) (width 0.2) (layer "F.Cu") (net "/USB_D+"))
 (segment (start 201.23241 71.23241) (end 201.5 71.5) (width 0.2) (layer "F.Cu") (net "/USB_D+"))
 (segment (start 200.5 70.58241) (end 200.76759 70.85) (width 0.2) (layer "F.Cu") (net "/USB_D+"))
 (segment (start 209.9 43.6) (end 208.3 42) (width 0.2) (layer "F.Cu") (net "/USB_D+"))
 (segment (start 200.5 69.825) (end 200.5 70.58241) (width 0.2) (layer "F.Cu") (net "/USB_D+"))
 (via (at 208 71.5) (size 0.6) (drill 0.3) (layers "F.Cu" "B.Cu") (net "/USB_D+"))
 (via (at 201.5 71.5) (size 0.6) (drill 0.3) (layers "F.Cu" "B.Cu") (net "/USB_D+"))
 (segment (start 202.09 72.09) (end 207.41 72.09) (width 0.2) (layer "B.Cu") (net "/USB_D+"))
 (segment (start 201.5 71.5) (end 202.09 72.09) (width 0.2) (layer "B.Cu") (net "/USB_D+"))
 (segment (start 207.41 72.09) (end 208 71.5) (width 0.2) (layer "B.Cu") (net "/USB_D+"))
 (segment (start 200.26759 68.8) (end 200.26759 66.23241) (width 0.2) (layer "F.Cu") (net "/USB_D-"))
 (segment (start 209.5 44.7) (end 208.3 43.5) (width 0.2) (layer "F.Cu") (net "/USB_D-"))
 (segment (start 200 69.06759) (end 200.26759 68.8) (width 0.2) (layer "F.Cu") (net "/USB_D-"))
 (segment (start 200.26759 66.23241) (end 200.5 66) (width 0.2) (layer "F.Cu") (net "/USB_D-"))
 (segment (start 200.26759 68.8) (end 200.73241 68.8) (width 0.2) (layer "F.Cu") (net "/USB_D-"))
 (segment (start 200.5 66) (end 201 66) (width 0.2) (layer "F.Cu") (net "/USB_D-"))
 (segment (start 209.5 65) (end 209.5 44.7) (width 0.2) (layer "F.Cu") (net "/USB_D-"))
 (segment (start 200 69.825) (end 200 69.06759) (width 0.2) (layer "F.Cu") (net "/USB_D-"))
 (segment (start 201 69.06759) (end 201 69.825) (width 0.2) (layer "F.Cu") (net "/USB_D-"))
 (segment (start 208.3 43.5) (end 208 43.5) (width 0.2) (layer "F.Cu") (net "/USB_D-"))
 (segment (start 200.73241 68.8) (end 201 69.06759) (width 0.2) (layer "F.Cu") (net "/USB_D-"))
 (segment (start 208.5 66) (end 209.5 65) (width 0.2) (layer "F.Cu") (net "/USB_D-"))
 (segment (start 208 66) (end 208.5 66) (width 0.2) (layer "F.Cu") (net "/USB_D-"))
 (via (at 201 66) (size 0.6) (drill 0.3) (layers "F.Cu" "B.Cu") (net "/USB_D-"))
 (via (at 208 66) (size 0.6) (drill 0.3) (layers "F.Cu" "B.Cu") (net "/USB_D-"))
 (segment (start 208 66) (end 201 66) (width 0.2) (layer "B.Cu") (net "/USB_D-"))
 (segment (start 202.5 68.21) (end 203.25 67.46) (width 0.2) (layer "F.Cu") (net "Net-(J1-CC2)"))
 (segment (start 202.5 69.825) (end 202.5 68.21) (width 0.2) (layer "F.Cu") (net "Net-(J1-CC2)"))
 (segment (start 190 39) (end 190.5 39) (width 0.2) (layer "F.Cu") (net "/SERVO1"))
 (segment (start 188.5 40.5) (end 190 39) (width 0.2) (layer "F.Cu") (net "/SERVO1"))
 (segment (start 183 74.5) (end 185.5 74.5) (width 0.2) (layer "F.Cu") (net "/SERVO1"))
 (segment (start 186 74) (end 186 73.1) (width 0.2) (layer "F.Cu") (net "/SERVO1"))
 (segment (start 185.5 74.5) (end 186 74) (width 0.2) (layer "F.Cu") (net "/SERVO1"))
 (via (at 186 74) (size 0.6) (drill 0.3) (layers "F.Cu" "B.Cu") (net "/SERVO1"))
 (via (at 186 73.1) (size 0.6) (drill 0.3) (layers "F.Cu" "B.Cu") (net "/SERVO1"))
 (via (at 188.5 40.5) (size 0.6) (drill 0.3) (layers "F.Cu" "B.Cu") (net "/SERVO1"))
 (segment (start 186 68) (end 188.5 65.5) (width 0.2) (layer "B.Cu") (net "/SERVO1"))
 (segment (start 188.5 65.5) (end 188.5 40.5) (width 0.2) (layer "B.Cu") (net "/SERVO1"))
 (segment (start 186 73.1) (end 186 68) (width 0.2) (layer "B.Cu") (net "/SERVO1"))
 (segment (start 185.5 39.5) (end 187.5 37.5) (width 0.5) (layer "F.Cu") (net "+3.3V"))
 (segment (start 184.9 48.5) (end 183.4 50) (width 0.5) (layer "F.Cu") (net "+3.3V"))
 (segment (start 182 52.5) (end 179.64259 52.5) (width 0.5) (layer "F.Cu") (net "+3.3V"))
 (segment (start 184.5 46) (end 184.5 39.5) (width 0.5) (layer "F.Cu") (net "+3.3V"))
 (segment (start 196.985 52.5) (end 186.5 52.5) (width 0.5) (layer "F.Cu") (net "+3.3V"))
 (segment (start 177.675 58.5) (end 177.675 54.46759) (width 0.5) (layer "F.Cu") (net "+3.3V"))
 (segment (start 186.5 52.5) (end 184.9 50.9) (width 0.5) (layer "F.Cu") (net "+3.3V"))
 (segment (start 178.3 51.15741) (end 178.3 50.7) (width 0.2) (layer "F.Cu") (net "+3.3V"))
 (segment (start 183.4 51.1) (end 182 52.5) (width 0.5) (layer "F.Cu") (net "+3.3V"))
 (segment (start 190.5 36) (end 189 36) (width 0.5) (layer "F.Cu") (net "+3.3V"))
 (segment (start 198.07 53.585) (end 196.985 52.5) (width 0.5) (layer "F.Cu") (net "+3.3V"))
 (segment (start 179.64259 52.5) (end 178.3 51.15741) (width 0.5) (layer "F.Cu") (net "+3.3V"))
 (segment (start 184.9 50.9) (end 184.9 48.5) (width 0.5) (layer "F.Cu") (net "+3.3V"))
 (segment (start 177.675 54.46759) (end 179.64259 52.5) (width 0.5) (layer "F.Cu") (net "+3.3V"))
 (segment (start 184.9 46.4) (end 184.5 46) (width 0.5) (layer "F.Cu") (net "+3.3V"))
 (segment (start 184.5 39.5) (end 185.5 39.5) (width 0.5) (layer "F.Cu") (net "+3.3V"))
 (segment (start 189 36) (end 187.5 37.5) (width 0.5) (layer "F.Cu") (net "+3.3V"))
 (segment (start 201.07 57.285) (end 201.07 56.07) (width 0.2) (layer "F.Cu") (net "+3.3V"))
 (segment (start 197 53.5) (end 197.985 53.5) (width 0.2) (layer "F.Cu") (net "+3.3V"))
 (segment (start 201.07 63.585) (end 201.07 57.285) (width 0.5) (layer "F.Cu") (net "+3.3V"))
 (segment (start 183.4 50) (end 183.4 51.1) (width 0.5) (layer "F.Cu") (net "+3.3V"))
 (segment (start 201.07 56.07) (end 201 56) (width 0.2) (layer "F.Cu") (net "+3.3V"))
 (segment (start 201 56) (end 201 55.60353) (width 0.2) (layer "F.Cu") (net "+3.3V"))
 (segment (start 201 55.60353) (end 201.051765 55.551765) (width 0.2) (layer "F.Cu") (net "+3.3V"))
 (segment (start 184.9 48.5) (end 184.9 46.4) (width 0.5) (layer "F.Cu") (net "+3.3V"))
 (segment (start 183.4 50) (end 181 50) (width 0.5) (layer "F.Cu") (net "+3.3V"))
 (segment (start 198.07 53.585) (end 197.985 53.5) (width 0.2) (layer "F.Cu") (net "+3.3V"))
 (via (at 197 53.5) (size 0.6) (drill 0.3) (layers "F.Cu" "B.Cu") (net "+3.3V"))
 (via (at 201.051765 55.551765) (size 0.6) (drill 0.3) (layers "F.Cu" "B.Cu") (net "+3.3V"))
 (segment (start 197 54.5) (end 197 53.5) (width 0.5) (layer "B.Cu") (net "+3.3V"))
 (segment (start 200 54.5) (end 197 54.5) (width 0.5) (layer "B.Cu") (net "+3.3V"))
 (segment (start 201.051765 55.551765) (end 200 54.5) (width 0.5) (layer "B.Cu") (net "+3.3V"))
 (segment (start 189.1 45.6) (end 185.478119 45.6) (width 0.2) (layer "F.Cu") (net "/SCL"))
 (segment (start 183.9 45.800003) (end 178.842587 45.800003) (width 0.2) (layer "F.Cu") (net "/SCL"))
 (segment (start 178.3 46.34259) (end 178.3 46.8) (width 0.2) (layer "F.Cu") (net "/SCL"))
 (segment (start 190.5 46.5) (end 190 46.5) (width 0.2) (layer "F.Cu") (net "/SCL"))
 (segment (start 190 46.5) (end 189.1 45.6) (width 0.2) (layer "F.Cu") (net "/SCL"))
 (segment (start 185.478119 45.6) (end 185.543761 45.665642) (width 0.2) (layer "F.Cu") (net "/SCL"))
 (segment (start 178.842587 45.800003) (end 178.3 46.34259) (width 0.2) (layer "F.Cu") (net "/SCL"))
 (via (at 183.9 45.800003) (size 0.6) (drill 0.3) (layers "F.Cu" "B.Cu") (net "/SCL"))
 (via (at 185.543761 45.665642) (size 0.6) (drill 0.3) (layers "F.Cu" "B.Cu") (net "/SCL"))
 (via (at 185.543761 45.665642) (size 0.6) (drill 0.3) (layers "F.Cu" "B.Cu") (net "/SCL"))
 (segment (start 184 45.700003) (end 183.9 45.800003) (width 0.2) (layer "B.Cu") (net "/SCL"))
 (segment (start 185.543761 45.665642) (end 185.478119 45.6) (width 0.2) (layer "B.Cu") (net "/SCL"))
 (segment (start 185.478119 45.6) (end 184 45.6) (width 0.2) (layer "B.Cu") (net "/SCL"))
 (segment (start 184 45.6) (end 184 45.700003) (width 0.2) (layer "B.Cu") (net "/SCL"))
 (segment (start 177.8 46.34259) (end 177.8 46.8) (width 0.2) (layer "F.Cu") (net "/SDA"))
 (segment (start 190.5 45) (end 185.1 45) (width 0.2) (layer "F.Cu") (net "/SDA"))
 (segment (start 178.5 45) (end 177.8 46.34259) (width 0.2) (layer "F.Cu") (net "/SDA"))
 (segment (start 183.9 45) (end 178.5 45) (width 0.2) (layer "F.Cu") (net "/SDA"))
 (via (at 185.1 45) (size 0.6) (drill 0.3) (layers "F.Cu" "B.Cu") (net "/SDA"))
 (via (at 183.9 45) (size 0.6) (drill 0.3) (layers "F.Cu" "B.Cu") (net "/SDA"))
 (segment (start 185.1 45) (end 183.9 45) (width 0.2) (layer "B.Cu") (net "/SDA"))
 (segment (start 176.1 44.4) (end 176.1 59.1) (width 0.2) (layer "F.Cu") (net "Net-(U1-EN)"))
 (segment (start 180.5 42) (end 181.5 43) (width 0.2) (layer "F.Cu") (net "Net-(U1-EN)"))
 (segment (start 189.1 37.5) (end 190.5 37.5) (width 0.2) (layer "F.Cu") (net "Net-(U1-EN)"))
 (segment (start 185.6 41) (end 189.1 37.5) (width 0.2) (layer "F.Cu") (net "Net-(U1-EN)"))
 (segment (start 185.6 42.9) (end 185.6 41) (width 0.2) (layer "F.Cu") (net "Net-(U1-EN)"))
 (segment (start 181.5 43.5) (end 181 44) (width 0.2) (layer "F.Cu") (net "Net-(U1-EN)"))
 (segment (start 181.5 43) (end 181.5 43.5) (width 0.2) (layer "F.Cu") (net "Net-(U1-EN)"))
 (segment (start 179 60) (end 179.5 59.5) (width 0.2) (layer "F.Cu") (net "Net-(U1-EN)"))
 (segment (start 177 60) (end 179 60) (width 0.2) (layer "F.Cu") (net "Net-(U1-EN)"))
 (segment (start 181.5 43) (end 183.9 43) (width 0.2) (layer "F.Cu") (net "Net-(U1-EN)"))
 (segment (start 181 44) (end 176.5 44) (width 0.2) (layer "F.Cu") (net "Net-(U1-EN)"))
 (segment (start 176.5 44) (end 176.1 44.4) (width 0.2) (layer "F.Cu") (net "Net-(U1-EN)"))
 (segment (start 176.1 59.1) (end 177 60) (width 0.2) (layer "F.Cu") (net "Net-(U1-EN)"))
 (segment (start 180.5 42) (end 180.5 36.75) (width 0.2) (layer "F.Cu") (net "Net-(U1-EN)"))
 (segment (start 179.5 59.5) (end 179.5 58.5) (width 0.2) (layer "F.Cu") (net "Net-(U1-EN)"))
 (segment (start 185.5 43) (end 185.6 42.9) (width 0.2) (layer "F.Cu") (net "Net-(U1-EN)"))
 (via (at 183.9 43) (size 0.6) (drill 0.3) (layers "F.Cu" "B.Cu") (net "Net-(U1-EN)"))
 (via (at 185.5 43) (size 0.6) (drill 0.3) (layers "F.Cu" "B.Cu") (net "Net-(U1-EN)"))
 (segment (start 183.9 43) (end 185.5 43) (width 0.2) (layer "B.Cu") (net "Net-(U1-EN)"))
 (segment (start 189 41.5) (end 189.1 41.5) (width 0.2) (layer "F.Cu") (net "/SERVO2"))
 (segment (start 184.6 65.5) (end 183 65.5) (width 0.2) (layer "F.Cu") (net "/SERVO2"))
 (segment (start 190 40.5) (end 189 41.5) (width 0.2) (layer "F.Cu") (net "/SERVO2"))
 (segment (start 189.1 61) (end 184.6 65.5) (width 0.2) (layer "F.Cu") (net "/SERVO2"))
 (segment (start 190.5 40.5) (end 190 40.5) (width 0.2) (layer "F.Cu") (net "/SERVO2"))
 (via (at 189.1 41.5) (size 0.6) (drill 0.3) (layers "F.Cu" "B.Cu") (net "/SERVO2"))
 (via (at 189.1 61) (size 0.6) (drill 0.3) (layers "F.Cu" "B.Cu") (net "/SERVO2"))
 (segment (start 189 61) (end 189.1 61) (width 0.2) (layer "B.Cu") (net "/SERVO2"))
 (segment (start 188.9 41.7) (end 188.9 60.9) (width 0.2) (layer "B.Cu") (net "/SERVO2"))
 (segment (start 189.1 41.5) (end 188.9 41.7) (width 0.2) (layer "B.Cu") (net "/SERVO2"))
 (segment (start 188.9 60.9) (end 189 61) (width 0.2) (layer "B.Cu") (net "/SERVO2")))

